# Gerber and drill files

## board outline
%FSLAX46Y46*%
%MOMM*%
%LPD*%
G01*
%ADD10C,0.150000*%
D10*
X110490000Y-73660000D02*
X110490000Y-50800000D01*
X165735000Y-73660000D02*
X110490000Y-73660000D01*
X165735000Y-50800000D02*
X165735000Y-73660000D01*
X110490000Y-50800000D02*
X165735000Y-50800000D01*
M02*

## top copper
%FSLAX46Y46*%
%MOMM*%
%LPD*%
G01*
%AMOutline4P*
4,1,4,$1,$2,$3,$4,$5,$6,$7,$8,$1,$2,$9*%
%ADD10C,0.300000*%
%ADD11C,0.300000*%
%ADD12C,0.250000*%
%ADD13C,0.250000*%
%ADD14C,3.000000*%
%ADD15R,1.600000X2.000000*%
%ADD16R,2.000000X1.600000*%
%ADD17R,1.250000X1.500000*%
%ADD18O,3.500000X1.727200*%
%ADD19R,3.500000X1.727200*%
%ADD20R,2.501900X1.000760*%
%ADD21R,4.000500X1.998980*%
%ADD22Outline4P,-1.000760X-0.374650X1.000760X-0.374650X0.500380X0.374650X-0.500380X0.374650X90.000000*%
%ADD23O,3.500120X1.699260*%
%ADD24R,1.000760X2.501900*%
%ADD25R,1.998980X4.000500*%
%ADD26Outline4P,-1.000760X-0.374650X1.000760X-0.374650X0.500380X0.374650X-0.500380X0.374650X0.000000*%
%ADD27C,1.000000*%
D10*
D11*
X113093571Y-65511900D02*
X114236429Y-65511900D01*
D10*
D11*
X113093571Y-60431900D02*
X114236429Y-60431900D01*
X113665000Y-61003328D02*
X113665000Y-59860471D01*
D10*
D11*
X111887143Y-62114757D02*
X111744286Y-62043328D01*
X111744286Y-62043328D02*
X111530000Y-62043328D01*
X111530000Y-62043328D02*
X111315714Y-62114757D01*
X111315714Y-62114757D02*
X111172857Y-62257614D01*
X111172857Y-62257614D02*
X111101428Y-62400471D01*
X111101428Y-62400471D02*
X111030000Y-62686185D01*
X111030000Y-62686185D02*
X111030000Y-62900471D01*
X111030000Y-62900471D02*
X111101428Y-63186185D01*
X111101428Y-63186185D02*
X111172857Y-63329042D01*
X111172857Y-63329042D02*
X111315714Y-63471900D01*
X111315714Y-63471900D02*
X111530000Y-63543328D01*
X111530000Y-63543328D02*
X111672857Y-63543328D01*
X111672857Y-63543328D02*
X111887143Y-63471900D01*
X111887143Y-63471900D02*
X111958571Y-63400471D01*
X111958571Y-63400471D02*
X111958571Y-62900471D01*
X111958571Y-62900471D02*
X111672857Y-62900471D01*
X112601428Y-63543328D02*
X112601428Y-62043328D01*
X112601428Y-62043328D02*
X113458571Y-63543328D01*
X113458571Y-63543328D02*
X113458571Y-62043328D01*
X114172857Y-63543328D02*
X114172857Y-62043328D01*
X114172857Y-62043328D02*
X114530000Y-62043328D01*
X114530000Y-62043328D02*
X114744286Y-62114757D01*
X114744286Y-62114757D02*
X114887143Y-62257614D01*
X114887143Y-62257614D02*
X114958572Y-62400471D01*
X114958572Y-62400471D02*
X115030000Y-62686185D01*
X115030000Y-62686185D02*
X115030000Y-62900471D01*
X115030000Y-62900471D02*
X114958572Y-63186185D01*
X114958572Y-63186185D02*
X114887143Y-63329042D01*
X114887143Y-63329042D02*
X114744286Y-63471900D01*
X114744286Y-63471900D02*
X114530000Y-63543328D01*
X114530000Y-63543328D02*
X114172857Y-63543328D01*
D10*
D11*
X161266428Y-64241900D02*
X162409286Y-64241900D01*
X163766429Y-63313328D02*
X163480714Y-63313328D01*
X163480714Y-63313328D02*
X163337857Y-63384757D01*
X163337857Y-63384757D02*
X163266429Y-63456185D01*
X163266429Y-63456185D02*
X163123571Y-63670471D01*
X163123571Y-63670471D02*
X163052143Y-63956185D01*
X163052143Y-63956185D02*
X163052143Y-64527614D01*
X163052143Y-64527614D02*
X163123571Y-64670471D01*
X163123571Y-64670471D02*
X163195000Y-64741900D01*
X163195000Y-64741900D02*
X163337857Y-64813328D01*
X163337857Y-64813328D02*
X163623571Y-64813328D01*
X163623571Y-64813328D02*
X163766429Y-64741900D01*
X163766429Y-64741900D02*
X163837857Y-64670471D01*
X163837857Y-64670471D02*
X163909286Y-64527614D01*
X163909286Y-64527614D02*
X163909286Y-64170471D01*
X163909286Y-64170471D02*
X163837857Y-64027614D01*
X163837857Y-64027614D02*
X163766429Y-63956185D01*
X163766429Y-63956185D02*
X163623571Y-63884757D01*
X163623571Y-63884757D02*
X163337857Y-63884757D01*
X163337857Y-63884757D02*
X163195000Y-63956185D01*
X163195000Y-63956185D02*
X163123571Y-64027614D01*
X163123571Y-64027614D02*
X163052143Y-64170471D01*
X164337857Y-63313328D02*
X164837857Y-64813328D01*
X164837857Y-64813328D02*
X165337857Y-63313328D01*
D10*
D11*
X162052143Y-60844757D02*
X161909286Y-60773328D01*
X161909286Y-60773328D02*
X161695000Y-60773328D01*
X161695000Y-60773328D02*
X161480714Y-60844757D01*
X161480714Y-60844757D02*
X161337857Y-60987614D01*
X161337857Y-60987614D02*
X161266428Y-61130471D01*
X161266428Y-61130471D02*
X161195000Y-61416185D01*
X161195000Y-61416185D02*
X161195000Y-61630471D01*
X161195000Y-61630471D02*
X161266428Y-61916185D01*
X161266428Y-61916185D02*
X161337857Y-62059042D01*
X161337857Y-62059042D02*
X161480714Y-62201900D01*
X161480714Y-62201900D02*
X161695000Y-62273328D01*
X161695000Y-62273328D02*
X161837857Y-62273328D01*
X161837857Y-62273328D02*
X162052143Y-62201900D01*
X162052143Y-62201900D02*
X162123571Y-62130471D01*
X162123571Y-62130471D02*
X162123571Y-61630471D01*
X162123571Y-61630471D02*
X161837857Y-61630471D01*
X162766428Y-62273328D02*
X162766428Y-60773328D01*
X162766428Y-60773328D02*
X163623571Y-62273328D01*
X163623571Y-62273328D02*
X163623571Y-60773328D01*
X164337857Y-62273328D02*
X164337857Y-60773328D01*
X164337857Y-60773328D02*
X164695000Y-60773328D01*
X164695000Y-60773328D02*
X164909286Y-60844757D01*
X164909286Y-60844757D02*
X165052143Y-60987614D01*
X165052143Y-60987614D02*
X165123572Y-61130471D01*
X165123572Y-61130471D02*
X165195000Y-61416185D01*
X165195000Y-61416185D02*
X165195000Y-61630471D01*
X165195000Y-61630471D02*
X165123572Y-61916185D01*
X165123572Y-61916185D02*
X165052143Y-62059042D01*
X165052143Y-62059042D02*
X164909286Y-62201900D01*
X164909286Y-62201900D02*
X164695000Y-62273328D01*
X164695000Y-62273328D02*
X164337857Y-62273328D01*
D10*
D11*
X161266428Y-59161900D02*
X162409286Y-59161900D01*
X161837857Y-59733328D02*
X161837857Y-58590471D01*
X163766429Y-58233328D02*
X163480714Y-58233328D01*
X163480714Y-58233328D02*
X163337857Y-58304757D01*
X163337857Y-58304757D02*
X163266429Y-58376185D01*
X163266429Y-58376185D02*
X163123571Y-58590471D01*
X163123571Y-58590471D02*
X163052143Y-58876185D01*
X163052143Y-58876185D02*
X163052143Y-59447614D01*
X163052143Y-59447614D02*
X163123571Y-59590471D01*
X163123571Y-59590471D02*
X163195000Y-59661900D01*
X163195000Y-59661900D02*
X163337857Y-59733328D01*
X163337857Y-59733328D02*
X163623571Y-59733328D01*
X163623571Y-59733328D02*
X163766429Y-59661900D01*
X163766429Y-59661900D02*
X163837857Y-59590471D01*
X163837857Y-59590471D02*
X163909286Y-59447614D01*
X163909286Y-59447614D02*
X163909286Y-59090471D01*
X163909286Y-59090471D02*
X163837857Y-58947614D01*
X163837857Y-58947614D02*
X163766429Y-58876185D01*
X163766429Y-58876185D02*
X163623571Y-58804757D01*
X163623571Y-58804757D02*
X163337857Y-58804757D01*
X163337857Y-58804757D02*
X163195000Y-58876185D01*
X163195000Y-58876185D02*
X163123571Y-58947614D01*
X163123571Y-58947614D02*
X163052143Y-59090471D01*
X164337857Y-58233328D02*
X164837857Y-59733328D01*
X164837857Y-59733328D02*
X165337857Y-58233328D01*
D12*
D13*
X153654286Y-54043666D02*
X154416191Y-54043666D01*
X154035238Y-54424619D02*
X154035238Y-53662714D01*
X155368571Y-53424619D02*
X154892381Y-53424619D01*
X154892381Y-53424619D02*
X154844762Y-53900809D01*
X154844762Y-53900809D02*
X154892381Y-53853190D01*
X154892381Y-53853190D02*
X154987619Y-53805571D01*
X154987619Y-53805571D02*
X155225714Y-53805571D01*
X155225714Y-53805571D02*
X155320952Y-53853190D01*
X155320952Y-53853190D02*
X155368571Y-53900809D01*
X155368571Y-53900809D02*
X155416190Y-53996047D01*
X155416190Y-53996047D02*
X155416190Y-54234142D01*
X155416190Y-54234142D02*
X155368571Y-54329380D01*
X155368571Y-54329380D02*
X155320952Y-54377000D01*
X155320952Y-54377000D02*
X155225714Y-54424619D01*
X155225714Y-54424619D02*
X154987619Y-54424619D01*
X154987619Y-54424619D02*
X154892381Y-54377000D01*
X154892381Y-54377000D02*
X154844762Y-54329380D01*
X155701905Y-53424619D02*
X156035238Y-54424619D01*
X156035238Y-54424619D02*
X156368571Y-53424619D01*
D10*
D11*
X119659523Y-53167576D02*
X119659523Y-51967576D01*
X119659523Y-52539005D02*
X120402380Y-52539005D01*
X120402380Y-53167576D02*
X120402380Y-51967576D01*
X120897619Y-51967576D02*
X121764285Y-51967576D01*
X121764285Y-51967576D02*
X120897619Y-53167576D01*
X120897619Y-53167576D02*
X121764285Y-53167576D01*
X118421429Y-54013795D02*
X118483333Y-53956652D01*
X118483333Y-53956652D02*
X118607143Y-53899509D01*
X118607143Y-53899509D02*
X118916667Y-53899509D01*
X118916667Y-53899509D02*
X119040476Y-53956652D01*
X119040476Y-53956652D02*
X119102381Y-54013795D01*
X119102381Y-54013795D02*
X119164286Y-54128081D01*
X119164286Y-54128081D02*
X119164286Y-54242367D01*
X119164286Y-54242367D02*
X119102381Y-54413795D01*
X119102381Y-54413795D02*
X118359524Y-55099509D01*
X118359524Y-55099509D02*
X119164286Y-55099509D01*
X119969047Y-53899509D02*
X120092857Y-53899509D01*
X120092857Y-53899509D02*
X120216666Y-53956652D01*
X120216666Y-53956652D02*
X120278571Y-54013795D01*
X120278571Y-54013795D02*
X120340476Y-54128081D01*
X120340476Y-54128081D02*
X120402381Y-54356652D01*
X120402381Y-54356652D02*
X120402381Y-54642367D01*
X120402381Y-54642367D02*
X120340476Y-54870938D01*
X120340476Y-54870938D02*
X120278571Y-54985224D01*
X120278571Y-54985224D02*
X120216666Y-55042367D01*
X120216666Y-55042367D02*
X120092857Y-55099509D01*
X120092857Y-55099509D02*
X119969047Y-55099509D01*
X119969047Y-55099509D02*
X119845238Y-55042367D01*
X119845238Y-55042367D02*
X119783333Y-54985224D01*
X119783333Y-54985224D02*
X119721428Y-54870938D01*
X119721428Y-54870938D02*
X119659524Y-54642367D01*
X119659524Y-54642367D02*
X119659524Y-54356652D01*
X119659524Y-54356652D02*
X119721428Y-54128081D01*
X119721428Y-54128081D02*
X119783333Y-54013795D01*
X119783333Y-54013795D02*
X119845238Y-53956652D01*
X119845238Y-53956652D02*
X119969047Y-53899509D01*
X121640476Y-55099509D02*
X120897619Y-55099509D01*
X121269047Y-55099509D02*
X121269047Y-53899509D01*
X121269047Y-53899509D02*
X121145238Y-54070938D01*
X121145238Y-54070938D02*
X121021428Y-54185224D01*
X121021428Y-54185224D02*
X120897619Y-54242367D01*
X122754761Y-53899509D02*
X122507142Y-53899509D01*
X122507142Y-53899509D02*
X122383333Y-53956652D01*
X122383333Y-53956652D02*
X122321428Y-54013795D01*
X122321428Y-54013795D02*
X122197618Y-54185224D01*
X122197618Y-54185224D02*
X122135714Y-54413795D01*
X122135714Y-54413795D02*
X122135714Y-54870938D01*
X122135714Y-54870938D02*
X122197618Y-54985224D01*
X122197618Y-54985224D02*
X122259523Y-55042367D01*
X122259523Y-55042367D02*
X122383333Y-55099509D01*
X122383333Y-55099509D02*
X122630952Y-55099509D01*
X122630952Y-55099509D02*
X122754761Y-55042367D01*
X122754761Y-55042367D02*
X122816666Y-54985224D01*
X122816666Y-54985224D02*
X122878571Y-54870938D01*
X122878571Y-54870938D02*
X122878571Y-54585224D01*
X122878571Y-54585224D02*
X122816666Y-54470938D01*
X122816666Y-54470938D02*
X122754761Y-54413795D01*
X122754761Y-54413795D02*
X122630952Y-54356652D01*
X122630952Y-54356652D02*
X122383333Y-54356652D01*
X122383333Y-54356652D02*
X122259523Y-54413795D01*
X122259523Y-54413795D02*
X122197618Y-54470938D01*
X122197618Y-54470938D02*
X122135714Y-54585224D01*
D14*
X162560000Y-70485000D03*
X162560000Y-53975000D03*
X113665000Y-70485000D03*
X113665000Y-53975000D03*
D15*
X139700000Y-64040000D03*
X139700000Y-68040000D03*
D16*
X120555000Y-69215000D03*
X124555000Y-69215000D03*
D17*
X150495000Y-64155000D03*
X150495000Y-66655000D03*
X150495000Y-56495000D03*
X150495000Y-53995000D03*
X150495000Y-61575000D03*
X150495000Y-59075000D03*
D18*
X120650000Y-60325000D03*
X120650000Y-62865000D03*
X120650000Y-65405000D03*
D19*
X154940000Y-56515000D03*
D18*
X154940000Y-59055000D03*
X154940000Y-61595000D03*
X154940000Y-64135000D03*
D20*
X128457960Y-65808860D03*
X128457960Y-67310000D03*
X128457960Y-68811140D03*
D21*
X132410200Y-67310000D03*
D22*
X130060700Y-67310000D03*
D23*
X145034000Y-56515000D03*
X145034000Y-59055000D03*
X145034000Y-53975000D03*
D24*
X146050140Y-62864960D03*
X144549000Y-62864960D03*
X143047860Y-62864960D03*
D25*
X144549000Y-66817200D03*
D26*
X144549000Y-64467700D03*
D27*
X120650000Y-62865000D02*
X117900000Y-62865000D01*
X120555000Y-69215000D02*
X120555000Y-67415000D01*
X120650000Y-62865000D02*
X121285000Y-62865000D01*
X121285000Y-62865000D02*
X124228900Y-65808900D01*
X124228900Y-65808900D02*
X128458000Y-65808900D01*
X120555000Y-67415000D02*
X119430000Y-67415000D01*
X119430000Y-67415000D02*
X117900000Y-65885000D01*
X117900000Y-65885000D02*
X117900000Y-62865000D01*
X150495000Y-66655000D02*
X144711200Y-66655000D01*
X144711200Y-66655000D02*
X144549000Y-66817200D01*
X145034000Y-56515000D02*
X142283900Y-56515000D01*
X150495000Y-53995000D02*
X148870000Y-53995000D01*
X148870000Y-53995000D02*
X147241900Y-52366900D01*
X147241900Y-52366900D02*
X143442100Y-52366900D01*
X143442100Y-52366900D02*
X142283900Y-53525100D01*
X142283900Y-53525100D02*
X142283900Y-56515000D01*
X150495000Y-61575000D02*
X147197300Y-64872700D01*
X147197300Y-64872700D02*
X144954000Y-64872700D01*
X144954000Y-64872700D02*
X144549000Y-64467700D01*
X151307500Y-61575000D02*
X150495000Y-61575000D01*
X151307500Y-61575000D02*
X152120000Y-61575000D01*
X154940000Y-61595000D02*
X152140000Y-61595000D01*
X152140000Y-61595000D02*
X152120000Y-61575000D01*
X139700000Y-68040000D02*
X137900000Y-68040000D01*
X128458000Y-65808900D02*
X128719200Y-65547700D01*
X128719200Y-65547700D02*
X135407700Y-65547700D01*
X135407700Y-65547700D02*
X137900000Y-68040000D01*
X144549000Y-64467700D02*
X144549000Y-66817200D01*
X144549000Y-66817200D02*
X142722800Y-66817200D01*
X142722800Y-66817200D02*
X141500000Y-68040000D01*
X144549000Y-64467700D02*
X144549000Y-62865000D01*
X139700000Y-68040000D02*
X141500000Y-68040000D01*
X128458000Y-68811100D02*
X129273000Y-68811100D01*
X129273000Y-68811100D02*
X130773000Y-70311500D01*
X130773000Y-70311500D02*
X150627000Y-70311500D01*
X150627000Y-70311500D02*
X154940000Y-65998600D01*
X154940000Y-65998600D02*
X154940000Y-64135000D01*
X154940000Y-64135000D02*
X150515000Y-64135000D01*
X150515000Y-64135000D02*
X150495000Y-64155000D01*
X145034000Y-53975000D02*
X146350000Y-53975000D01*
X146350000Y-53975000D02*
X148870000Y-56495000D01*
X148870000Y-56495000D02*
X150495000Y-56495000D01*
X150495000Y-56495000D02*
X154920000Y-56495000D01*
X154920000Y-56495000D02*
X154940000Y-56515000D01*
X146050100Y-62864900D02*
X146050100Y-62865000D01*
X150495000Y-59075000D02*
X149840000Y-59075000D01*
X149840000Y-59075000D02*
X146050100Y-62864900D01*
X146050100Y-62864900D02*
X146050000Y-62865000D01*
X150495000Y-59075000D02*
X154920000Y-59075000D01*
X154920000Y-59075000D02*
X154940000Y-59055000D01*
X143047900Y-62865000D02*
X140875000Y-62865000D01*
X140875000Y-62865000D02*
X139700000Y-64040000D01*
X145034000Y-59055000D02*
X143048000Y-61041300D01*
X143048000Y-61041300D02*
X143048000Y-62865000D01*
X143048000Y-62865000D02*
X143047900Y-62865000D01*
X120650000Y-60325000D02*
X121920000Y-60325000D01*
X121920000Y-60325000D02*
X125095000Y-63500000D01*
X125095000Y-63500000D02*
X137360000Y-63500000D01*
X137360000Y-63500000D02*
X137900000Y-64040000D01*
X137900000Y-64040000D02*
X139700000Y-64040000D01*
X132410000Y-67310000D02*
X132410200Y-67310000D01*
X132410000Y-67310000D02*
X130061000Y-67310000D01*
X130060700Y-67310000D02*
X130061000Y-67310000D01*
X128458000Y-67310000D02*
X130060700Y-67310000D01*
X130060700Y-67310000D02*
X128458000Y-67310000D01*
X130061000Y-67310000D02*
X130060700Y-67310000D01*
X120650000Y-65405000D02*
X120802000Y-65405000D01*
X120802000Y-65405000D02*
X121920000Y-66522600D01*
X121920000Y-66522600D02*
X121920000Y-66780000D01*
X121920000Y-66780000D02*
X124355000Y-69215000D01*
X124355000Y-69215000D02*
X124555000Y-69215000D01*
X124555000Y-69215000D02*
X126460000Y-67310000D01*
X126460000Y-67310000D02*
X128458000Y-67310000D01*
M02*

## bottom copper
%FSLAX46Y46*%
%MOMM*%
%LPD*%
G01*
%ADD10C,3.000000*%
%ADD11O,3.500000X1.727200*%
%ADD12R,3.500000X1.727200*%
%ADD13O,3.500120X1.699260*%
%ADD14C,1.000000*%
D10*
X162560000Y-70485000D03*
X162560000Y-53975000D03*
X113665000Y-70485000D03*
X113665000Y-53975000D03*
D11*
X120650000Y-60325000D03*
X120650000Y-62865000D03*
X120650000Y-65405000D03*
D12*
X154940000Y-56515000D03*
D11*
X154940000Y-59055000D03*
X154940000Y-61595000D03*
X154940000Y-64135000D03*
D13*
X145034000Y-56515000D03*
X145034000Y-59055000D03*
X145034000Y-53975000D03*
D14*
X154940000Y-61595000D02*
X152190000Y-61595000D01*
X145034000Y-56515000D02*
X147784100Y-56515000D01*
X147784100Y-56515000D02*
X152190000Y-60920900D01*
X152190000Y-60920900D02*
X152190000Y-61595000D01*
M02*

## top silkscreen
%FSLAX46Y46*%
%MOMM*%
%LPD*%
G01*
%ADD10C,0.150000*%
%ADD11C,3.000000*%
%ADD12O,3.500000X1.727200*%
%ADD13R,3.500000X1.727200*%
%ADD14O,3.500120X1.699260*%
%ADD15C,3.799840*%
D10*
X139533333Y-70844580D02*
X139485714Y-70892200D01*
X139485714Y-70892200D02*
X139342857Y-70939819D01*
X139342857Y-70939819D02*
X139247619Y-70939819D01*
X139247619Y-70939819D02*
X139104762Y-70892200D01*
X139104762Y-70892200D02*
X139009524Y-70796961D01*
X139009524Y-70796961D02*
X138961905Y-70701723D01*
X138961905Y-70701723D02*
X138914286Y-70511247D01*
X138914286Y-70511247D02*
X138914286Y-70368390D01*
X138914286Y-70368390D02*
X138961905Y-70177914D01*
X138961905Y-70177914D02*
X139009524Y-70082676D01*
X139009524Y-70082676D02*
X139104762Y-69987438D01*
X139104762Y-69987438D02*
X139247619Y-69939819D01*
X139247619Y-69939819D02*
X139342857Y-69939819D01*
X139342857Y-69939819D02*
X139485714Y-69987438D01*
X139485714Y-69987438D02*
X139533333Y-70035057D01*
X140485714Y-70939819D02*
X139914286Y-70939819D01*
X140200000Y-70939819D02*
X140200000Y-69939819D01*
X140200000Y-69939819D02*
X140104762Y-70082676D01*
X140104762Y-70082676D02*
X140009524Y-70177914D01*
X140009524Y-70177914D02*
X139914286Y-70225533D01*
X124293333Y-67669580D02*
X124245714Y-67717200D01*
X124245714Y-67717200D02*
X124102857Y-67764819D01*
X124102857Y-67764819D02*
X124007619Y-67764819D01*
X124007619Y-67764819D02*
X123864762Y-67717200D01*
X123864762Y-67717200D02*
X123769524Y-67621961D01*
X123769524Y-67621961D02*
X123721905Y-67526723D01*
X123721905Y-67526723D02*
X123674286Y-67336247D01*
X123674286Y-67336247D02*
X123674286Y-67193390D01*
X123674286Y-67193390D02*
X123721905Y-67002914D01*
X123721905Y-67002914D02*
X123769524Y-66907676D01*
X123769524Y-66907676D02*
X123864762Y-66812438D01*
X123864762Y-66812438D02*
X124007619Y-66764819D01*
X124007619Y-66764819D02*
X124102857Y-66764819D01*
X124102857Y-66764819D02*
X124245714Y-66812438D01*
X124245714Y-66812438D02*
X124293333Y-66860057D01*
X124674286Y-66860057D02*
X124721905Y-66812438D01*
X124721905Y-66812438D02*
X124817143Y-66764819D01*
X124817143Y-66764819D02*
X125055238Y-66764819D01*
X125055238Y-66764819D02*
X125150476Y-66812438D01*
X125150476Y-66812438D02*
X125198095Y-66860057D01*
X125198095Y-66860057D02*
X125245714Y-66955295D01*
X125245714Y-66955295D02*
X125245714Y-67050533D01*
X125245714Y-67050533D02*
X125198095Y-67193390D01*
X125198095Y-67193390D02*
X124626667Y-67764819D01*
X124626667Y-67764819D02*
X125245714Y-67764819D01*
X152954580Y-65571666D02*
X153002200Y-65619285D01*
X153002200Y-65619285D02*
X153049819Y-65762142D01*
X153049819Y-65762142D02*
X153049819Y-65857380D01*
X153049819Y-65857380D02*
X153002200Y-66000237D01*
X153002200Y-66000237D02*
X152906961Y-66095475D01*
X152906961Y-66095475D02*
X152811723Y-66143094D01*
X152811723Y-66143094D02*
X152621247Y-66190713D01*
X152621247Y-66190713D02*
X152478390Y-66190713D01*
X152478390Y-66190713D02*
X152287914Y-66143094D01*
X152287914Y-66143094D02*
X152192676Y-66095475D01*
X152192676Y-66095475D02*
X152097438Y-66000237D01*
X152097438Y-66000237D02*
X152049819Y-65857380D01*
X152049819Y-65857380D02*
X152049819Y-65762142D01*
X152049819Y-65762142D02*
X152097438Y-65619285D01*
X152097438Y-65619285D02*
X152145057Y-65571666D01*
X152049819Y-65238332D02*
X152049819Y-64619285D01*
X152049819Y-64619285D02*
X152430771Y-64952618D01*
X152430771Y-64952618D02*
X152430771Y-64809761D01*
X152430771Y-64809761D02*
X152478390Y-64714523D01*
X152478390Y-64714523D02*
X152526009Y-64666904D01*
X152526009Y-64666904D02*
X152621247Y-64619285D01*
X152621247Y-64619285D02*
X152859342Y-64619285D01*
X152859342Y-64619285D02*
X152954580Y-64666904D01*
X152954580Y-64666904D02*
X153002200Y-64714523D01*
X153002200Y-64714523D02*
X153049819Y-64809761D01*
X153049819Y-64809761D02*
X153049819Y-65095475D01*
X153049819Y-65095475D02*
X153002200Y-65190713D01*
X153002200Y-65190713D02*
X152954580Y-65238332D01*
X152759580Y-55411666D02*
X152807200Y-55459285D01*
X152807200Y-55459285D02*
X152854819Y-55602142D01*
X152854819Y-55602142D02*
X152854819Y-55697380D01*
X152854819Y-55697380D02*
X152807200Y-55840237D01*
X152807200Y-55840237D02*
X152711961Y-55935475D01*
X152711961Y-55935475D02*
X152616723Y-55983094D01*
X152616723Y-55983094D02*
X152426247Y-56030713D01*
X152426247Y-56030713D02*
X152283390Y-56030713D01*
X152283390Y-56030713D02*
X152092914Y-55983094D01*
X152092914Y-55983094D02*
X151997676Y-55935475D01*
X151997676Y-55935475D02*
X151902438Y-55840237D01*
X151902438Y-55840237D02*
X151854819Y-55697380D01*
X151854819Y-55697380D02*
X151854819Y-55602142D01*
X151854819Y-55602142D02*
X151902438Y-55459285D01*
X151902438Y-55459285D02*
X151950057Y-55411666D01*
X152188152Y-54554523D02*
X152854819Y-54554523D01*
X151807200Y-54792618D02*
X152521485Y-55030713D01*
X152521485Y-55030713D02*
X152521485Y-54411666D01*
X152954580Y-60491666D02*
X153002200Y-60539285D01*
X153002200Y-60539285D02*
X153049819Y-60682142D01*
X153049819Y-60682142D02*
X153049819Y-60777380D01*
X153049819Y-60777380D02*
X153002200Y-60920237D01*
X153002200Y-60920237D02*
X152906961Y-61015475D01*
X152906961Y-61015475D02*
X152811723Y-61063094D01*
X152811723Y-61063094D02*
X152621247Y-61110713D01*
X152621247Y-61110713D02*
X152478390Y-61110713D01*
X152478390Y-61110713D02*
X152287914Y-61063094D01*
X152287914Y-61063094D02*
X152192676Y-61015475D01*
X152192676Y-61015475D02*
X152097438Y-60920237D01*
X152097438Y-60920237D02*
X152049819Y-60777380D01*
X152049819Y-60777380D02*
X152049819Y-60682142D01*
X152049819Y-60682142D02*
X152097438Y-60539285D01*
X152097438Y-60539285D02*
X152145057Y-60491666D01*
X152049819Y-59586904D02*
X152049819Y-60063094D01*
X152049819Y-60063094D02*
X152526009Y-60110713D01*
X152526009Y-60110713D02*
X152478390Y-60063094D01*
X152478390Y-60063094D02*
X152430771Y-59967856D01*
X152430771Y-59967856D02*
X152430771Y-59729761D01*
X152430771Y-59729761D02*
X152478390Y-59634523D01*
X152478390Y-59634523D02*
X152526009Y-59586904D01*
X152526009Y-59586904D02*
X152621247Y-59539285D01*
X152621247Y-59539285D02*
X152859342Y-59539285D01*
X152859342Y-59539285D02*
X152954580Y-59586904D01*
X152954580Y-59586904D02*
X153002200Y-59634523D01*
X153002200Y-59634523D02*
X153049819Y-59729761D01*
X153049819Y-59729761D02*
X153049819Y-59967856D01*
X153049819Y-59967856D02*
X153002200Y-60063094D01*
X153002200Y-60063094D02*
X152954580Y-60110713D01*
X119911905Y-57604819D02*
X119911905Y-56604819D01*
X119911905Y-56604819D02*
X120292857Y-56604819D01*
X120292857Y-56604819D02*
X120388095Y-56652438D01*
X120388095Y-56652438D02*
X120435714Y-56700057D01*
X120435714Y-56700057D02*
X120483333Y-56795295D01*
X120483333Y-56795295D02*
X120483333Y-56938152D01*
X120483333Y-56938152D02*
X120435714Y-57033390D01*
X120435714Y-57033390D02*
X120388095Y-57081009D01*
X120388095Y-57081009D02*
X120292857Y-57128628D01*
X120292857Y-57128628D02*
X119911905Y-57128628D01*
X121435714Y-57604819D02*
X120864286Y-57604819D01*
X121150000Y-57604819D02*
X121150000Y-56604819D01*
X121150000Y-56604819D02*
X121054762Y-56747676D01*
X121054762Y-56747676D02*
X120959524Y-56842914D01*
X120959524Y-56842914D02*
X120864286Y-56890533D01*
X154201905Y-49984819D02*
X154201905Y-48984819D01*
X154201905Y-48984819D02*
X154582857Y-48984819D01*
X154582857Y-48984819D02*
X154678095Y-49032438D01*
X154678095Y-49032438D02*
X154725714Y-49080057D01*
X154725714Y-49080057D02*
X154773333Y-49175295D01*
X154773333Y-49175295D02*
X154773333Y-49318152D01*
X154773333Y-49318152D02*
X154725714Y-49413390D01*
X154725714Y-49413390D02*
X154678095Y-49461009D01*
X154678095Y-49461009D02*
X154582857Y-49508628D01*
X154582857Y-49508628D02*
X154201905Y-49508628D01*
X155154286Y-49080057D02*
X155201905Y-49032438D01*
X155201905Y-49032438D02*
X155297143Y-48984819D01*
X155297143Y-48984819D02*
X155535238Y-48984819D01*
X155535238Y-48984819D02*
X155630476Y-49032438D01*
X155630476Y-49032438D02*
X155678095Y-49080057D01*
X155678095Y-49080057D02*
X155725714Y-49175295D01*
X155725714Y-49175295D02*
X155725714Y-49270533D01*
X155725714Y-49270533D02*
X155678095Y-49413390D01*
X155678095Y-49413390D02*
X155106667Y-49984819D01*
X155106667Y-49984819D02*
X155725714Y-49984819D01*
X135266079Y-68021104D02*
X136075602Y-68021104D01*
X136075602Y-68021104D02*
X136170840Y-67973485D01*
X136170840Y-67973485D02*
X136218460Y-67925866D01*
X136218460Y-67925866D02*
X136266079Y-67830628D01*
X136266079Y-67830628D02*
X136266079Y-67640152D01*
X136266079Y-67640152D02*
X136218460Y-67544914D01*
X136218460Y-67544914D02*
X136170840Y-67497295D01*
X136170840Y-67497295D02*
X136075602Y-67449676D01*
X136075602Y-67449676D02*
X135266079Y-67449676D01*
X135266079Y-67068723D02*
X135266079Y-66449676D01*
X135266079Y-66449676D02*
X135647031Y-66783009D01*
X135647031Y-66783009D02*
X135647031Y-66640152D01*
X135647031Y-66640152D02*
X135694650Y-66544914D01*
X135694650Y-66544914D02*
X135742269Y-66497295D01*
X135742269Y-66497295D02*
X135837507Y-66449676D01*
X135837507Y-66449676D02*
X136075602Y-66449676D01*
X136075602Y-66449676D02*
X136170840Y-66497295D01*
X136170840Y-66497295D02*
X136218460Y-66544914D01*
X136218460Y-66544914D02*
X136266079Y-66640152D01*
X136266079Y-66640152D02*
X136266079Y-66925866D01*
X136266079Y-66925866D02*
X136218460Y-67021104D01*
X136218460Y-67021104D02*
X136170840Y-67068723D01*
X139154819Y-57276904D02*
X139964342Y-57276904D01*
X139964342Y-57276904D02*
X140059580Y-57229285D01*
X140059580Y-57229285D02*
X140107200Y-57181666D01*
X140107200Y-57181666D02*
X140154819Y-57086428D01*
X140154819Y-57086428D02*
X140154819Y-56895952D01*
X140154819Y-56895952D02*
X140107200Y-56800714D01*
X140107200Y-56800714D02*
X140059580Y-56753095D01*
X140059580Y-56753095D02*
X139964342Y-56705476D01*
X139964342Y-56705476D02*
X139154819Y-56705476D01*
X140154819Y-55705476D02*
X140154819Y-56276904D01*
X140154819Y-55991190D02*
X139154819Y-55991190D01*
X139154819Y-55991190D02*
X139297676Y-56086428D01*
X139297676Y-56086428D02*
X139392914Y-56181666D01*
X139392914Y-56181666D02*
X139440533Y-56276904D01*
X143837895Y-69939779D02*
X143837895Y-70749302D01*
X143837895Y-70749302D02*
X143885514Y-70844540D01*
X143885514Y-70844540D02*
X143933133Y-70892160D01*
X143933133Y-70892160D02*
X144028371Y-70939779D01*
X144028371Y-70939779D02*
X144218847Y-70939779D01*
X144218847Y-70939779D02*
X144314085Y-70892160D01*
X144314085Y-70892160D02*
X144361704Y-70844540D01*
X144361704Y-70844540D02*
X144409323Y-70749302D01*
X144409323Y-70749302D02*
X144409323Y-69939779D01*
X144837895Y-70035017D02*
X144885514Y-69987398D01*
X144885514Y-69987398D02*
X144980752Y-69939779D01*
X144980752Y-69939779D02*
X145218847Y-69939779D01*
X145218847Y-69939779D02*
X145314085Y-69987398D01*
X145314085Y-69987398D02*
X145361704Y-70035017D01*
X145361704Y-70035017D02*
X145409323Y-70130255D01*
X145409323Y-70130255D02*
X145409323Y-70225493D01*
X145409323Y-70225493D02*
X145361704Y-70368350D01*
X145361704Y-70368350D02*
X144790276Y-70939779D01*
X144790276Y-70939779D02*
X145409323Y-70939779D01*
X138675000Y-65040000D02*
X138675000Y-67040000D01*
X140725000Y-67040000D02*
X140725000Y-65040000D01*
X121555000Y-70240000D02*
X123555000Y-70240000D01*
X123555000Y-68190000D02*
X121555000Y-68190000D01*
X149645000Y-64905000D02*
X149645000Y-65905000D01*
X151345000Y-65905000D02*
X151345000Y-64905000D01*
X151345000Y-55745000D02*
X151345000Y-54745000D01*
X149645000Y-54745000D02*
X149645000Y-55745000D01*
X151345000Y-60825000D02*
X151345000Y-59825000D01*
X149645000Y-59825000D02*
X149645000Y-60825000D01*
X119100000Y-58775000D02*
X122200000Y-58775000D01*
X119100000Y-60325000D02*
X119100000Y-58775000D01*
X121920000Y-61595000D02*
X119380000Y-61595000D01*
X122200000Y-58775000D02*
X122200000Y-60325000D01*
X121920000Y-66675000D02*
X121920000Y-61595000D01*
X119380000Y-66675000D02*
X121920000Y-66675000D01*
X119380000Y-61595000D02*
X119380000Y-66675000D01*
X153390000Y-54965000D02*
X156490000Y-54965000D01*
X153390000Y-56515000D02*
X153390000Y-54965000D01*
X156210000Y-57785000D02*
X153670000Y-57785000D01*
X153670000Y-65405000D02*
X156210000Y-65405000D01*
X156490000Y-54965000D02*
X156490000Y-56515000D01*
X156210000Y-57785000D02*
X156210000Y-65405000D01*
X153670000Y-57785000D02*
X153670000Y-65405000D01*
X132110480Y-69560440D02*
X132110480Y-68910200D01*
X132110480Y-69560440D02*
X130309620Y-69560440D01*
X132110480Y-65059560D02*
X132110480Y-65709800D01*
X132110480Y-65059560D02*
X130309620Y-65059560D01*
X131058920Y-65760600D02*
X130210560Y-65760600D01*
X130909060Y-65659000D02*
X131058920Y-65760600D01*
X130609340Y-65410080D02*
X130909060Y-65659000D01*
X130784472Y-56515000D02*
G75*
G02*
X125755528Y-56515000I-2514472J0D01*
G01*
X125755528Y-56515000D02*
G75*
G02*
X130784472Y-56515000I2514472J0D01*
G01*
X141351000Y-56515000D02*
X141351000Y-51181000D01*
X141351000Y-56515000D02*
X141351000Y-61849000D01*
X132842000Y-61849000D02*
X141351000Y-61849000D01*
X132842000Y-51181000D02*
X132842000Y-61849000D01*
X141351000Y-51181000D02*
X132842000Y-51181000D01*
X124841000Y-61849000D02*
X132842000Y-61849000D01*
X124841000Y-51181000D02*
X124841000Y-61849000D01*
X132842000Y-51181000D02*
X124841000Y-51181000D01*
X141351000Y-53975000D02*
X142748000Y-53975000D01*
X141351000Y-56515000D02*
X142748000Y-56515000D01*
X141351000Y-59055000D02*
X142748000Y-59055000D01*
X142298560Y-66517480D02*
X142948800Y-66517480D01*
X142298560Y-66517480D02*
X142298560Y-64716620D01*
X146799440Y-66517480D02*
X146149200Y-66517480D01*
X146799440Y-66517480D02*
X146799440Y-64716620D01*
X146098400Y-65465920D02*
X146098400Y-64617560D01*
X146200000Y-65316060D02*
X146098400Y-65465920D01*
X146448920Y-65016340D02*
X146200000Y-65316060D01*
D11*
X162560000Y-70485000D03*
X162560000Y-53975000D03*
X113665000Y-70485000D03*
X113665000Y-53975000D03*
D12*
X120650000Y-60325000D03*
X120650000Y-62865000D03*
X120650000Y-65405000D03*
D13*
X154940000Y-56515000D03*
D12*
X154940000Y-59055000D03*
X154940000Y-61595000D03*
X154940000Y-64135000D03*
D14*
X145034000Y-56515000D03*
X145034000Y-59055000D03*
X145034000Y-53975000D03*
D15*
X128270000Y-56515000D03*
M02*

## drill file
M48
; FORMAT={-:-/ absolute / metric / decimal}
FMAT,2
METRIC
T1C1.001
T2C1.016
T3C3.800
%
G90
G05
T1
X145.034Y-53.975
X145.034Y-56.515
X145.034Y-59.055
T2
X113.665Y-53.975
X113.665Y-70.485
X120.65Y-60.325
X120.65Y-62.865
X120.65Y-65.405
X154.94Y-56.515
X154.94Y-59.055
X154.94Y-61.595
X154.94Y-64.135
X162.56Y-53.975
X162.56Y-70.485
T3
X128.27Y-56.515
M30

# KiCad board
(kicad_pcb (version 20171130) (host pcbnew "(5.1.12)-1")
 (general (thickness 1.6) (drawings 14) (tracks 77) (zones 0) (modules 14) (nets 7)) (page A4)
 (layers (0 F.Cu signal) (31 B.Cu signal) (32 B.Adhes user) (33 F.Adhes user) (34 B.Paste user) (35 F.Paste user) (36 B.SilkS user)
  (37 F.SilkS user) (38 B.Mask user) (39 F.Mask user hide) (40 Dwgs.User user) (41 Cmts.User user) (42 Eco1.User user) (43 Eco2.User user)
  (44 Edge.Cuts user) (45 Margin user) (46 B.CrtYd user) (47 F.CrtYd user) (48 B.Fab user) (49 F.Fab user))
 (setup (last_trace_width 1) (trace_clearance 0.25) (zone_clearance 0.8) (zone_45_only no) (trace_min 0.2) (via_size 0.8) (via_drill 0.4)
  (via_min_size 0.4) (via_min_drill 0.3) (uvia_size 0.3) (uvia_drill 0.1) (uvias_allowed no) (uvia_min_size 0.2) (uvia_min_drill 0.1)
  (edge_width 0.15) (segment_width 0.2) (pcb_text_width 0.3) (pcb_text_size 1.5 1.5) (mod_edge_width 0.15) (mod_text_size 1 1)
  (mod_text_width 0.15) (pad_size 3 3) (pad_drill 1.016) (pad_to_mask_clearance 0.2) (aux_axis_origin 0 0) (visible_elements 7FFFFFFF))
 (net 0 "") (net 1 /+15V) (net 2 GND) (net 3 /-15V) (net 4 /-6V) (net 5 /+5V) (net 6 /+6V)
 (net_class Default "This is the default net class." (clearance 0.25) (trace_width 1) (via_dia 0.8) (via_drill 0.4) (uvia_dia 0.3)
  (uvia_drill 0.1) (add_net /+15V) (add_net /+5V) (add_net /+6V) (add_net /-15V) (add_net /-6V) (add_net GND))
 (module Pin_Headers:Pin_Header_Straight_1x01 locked (layer F.Cu) (at 162.56 70.485)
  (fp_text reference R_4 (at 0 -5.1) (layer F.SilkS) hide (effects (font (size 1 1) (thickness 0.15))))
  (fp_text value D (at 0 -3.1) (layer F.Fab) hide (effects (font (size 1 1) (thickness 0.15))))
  (pad 1 thru_hole circle (at 0 0) (size 3 3) (drill 1.016) (layers *.Cu *.Mask F.SilkS)))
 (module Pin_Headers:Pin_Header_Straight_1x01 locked (layer F.Cu) (at 162.56 53.975)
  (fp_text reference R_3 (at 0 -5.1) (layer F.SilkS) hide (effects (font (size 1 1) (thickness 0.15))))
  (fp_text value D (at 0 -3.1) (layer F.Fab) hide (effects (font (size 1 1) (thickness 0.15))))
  (pad 1 thru_hole circle (at 0 0) (size 3 3) (drill 1.016) (layers *.Cu *.Mask F.SilkS)))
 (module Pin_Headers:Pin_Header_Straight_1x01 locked (layer F.Cu) (at 113.665 70.485)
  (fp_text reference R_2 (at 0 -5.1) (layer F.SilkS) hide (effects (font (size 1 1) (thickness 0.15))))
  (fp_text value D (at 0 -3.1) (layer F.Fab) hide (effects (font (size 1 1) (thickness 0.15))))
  (pad 1 thru_hole circle (at 0 0) (size 3 3) (drill 1.016) (layers *.Cu *.Mask F.SilkS)))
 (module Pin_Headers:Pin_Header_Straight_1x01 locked (layer F.Cu) (at 113.665 53.975)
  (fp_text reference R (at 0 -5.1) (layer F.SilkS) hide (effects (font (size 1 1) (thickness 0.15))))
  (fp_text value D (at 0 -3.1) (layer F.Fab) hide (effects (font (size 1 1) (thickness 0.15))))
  (pad 1 thru_hole circle (at 0 0) (size 3 3) (drill 1.016) (layers *.Cu *.Mask F.SilkS)))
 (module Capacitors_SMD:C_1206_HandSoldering (layer F.Cu) (at 139.7 66.04 270)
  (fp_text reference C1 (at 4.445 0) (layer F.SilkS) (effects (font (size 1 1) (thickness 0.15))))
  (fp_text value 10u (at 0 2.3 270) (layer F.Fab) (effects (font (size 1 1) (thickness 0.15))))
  (fp_line (start -1 1.025) (end 1 1.025) (layer F.SilkS) (width 0.15))
  (fp_line (start 1 -1.025) (end -1 -1.025) (layer F.SilkS) (width 0.15))
  (pad 1 smd rect (at -2 0 270) (size 2 1.6) (layers F.Cu F.Paste F.Mask) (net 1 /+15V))
  (pad 2 smd rect (at 2 0 270) (size 2 1.6) (layers F.Cu F.Paste F.Mask) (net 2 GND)))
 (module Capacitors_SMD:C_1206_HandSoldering (layer F.Cu) (at 122.555 69.215 180)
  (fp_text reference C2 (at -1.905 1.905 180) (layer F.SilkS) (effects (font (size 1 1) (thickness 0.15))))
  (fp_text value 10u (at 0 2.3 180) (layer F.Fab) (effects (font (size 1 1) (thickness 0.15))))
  (fp_line (start 1 -1.025) (end -1 -1.025) (layer F.SilkS) (width 0.15))
  (fp_line (start -1 1.025) (end 1 1.025) (layer F.SilkS) (width 0.15))
  (pad 2 smd rect (at 2 0 180) (size 2 1.6) (layers F.Cu F.Paste F.Mask) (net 2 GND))
  (pad 1 smd rect (at -2 0 180) (size 2 1.6) (layers F.Cu F.Paste F.Mask) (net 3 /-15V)))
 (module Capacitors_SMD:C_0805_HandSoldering (layer F.Cu) (at 150.495 65.405 270)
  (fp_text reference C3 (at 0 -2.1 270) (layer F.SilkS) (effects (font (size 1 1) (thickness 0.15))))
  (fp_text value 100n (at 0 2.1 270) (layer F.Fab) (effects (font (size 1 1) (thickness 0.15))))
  (fp_line (start -0.5 0.85) (end 0.5 0.85) (layer F.SilkS) (width 0.15))
  (fp_line (start 0.5 -0.85) (end -0.5 -0.85) (layer F.SilkS) (width 0.15))
  (pad 1 smd rect (at -1.25 0 270) (size 1.5 1.25) (layers F.Cu F.Paste F.Mask) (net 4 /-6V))
  (pad 2 smd rect (at 1.25 0 270) (size 1.5 1.25) (layers F.Cu F.Paste F.Mask) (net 2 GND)))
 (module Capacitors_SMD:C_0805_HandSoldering (layer F.Cu) (at 150.495 55.245 90)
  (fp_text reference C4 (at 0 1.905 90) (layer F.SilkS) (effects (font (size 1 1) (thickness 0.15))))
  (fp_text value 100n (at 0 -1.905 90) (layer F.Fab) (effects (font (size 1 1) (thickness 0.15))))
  (fp_line (start -0.5 0.85) (end 0.5 0.85) (layer F.SilkS) (width 0.15))
  (fp_line (start 0.5 -0.85) (end -0.5 -0.85) (layer F.SilkS) (width 0.15))
  (pad 1 smd rect (at -1.25 0 90) (size 1.5 1.25) (layers F.Cu F.Paste F.Mask) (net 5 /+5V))
  (pad 2 smd rect (at 1.25 0 90) (size 1.5 1.25) (layers F.Cu F.Paste F.Mask) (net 2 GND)))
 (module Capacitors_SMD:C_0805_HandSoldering (layer F.Cu) (at 150.495 60.325 270)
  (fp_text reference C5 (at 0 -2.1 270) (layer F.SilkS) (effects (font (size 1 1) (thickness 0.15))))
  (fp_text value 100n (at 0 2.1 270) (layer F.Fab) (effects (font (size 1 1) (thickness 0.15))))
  (fp_line (start 0.5 -0.85) (end -0.5 -0.85) (layer F.SilkS) (width 0.15))
  (fp_line (start -0.5 0.85) (end 0.5 0.85) (layer F.SilkS) (width 0.15))
  (pad 2 smd rect (at 1.25 0 270) (size 1.5 1.25) (layers F.Cu F.Paste F.Mask) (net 2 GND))
  (pad 1 smd rect (at -1.25 0 270) (size 1.5 1.25) (layers F.Cu F.Paste F.Mask) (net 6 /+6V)))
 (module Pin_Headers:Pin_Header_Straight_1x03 (layer F.Cu) (at 120.65 60.325)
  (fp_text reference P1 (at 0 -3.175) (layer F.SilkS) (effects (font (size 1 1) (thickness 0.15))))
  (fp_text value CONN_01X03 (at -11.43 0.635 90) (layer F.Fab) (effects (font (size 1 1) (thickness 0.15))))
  (fp_line (start -1.55 -1.55) (end 1.55 -1.55) (layer F.SilkS) (width 0.15))
  (fp_line (start -1.55 0) (end -1.55 -1.55) (layer F.SilkS) (width 0.15))
  (fp_line (start 1.27 1.27) (end -1.27 1.27) (layer F.SilkS) (width 0.15))
  (fp_line (start 1.55 -1.55) (end 1.55 0) (layer F.SilkS) (width 0.15))
  (fp_line (start 1.27 6.35) (end 1.27 1.27) (layer F.SilkS) (width 0.15))
  (fp_line (start -1.27 6.35) (end 1.27 6.35) (layer F.SilkS) (width 0.15))
  (fp_line (start -1.27 1.27) (end -1.27 6.35) (layer F.SilkS) (width 0.15))
  (pad 1 thru_hole oval (at 0 0) (size 3.5 1.7272) (drill 1.016) (layers *.Cu *.Mask F.SilkS) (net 1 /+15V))
  (pad 2 thru_hole oval (at 0 2.54) (size 3.5 1.7272) (drill 1.016) (layers *.Cu *.Mask F.SilkS) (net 2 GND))
  (pad 3 thru_hole oval (at 0 5.08) (size 3.5 1.7272) (drill 1.016) (layers *.Cu *.Mask F.SilkS) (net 3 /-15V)))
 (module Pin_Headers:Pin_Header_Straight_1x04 (layer F.Cu) (at 154.94 56.515)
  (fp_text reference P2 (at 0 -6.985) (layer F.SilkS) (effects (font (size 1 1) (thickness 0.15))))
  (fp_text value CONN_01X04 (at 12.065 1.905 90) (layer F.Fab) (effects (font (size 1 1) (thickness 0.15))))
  (fp_line (start -1.55 -1.55) (end 1.55 -1.55) (layer F.SilkS) (width 0.15))
  (fp_line (start -1.55 0) (end -1.55 -1.55) (layer F.SilkS) (width 0.15))
  (fp_line (start 1.27 1.27) (end -1.27 1.27) (layer F.SilkS) (width 0.15))
  (fp_line (start -1.27 8.89) (end 1.27 8.89) (layer F.SilkS) (width 0.15))
  (fp_line (start 1.55 -1.55) (end 1.55 0) (layer F.SilkS) (width 0.15))
  (fp_line (start 1.27 1.27) (end 1.27 8.89) (layer F.SilkS) (width 0.15))
  (fp_line (start -1.27 1.27) (end -1.27 8.89) (layer F.SilkS) (width 0.15))
  (pad 1 thru_hole rect (at 0 0) (size 3.5 1.7272) (drill 1.016) (layers *.Cu *.Mask F.SilkS) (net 5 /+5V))
  (pad 2 thru_hole oval (at 0 2.54) (size 3.5 1.7272) (drill 1.016) (layers *.Cu *.Mask F.SilkS) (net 6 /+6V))
  (pad 3 thru_hole oval (at 0 5.08) (size 3.5 1.7272) (drill 1.016) (layers *.Cu *.Mask F.SilkS) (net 2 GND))
  (pad 4 thru_hole oval (at 0 7.62) (size 3.5 1.7272) (drill 1.016) (layers *.Cu *.Mask F.SilkS) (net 4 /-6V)))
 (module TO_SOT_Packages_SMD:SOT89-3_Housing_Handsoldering (layer F.Cu) (at 130.81 67.31 270)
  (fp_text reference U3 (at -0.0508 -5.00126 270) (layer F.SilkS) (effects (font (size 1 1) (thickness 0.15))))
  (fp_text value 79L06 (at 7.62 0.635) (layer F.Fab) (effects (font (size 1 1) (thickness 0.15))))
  (fp_line (start 2.25044 -1.30048) (end 1.6002 -1.30048) (layer F.SilkS) (width 0.15))
  (fp_line (start 2.25044 -1.30048) (end 2.25044 0.50038) (layer F.SilkS) (width 0.15))
  (fp_line (start -2.25044 -1.30048) (end -1.6002 -1.30048) (layer F.SilkS) (width 0.15))
  (fp_line (start -2.25044 -1.30048) (end -2.25044 0.50038) (layer F.SilkS) (width 0.15))
  (fp_line (start -1.5494 -0.24892) (end -1.5494 0.59944) (layer F.SilkS) (width 0.15))
  (fp_line (start -1.651 -0.09906) (end -1.5494 -0.24892) (layer F.SilkS) (width 0.15))
  (fp_line (start -1.89992 0.20066) (end -1.651 -0.09906) (layer F.SilkS) (width 0.15))
  (pad 1 smd rect (at -1.50114 2.35204 270) (size 1.00076 2.5019) (layers F.Cu F.Paste F.Mask) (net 2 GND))
  (pad 2 smd rect (at 0 2.35204 270) (size 1.00076 2.5019) (layers F.Cu F.Paste F.Mask) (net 3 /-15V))
  (pad 3 smd rect (at 1.50114 2.35204 270) (size 1.00076 2.5019) (layers F.Cu F.Paste F.Mask) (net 4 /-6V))
  (pad 2 smd rect (at 0 -1.6002 270) (size 1.99898 4.0005) (layers F.Cu F.Paste F.Mask) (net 3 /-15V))
  (pad 2 smd trapezoid (at 0 0.7493 90) (size 1.50114 0.7493) (rect_delta 0 0.50038) (layers F.Cu F.Paste F.Mask) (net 3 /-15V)))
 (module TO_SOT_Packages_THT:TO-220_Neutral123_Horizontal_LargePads (layer F.Cu) (at 145.034 56.515 90)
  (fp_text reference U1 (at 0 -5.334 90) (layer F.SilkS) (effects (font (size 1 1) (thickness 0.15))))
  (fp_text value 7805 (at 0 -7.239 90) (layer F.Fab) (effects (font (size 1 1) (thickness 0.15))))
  (fp_circle (center 0 -16.764) (end 1.778 -14.986) (layer F.SilkS) (width 0.15))
  (fp_line (start 0 -3.683) (end 5.334 -3.683) (layer F.SilkS) (width 0.15))
  (fp_line (start 0 -3.683) (end -5.334 -3.683) (layer F.SilkS) (width 0.15))
  (fp_line (start -5.334 -12.192) (end -5.334 -3.683) (layer F.SilkS) (width 0.15))
  (fp_line (start 5.334 -12.192) (end -5.334 -12.192) (layer F.SilkS) (width 0.15))
  (fp_line (start 5.334 -3.683) (end 5.334 -12.192) (layer F.SilkS) (width 0.15))
  (fp_line (start -5.334 -20.193) (end -5.334 -12.192) (layer F.SilkS) (width 0.15))
  (fp_line (start 5.334 -20.193) (end -5.334 -20.193) (layer F.SilkS) (width 0.15))
  (fp_line (start 5.334 -12.192) (end 5.334 -20.193) (layer F.SilkS) (width 0.15))
  (fp_line (start 2.54 -3.683) (end 2.54 -2.286) (layer F.SilkS) (width 0.15))
  (fp_line (start 0 -3.683) (end 0 -2.286) (layer F.SilkS) (width 0.15))
  (fp_line (start -2.54 -3.683) (end -2.54 -2.286) (layer F.SilkS) (width 0.15))
  (pad 2 thru_hole oval (at 0 0 180) (size 3.50012 1.69926) (drill 1.00076) (layers *.Cu *.Mask F.SilkS) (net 2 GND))
  (pad 1 thru_hole oval (at -2.54 0 180) (size 3.50012 1.69926) (drill 1.00076) (layers *.Cu *.Mask F.SilkS) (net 1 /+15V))
  (pad 3 thru_hole oval (at 2.54 0 180) (size 3.50012 1.69926) (drill 1.00076) (layers *.Cu *.Mask F.SilkS) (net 5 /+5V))
  (pad "" np_thru_hole circle (at 0 -16.764 180) (size 3.79984 3.79984) (drill 3.79984) (layers *.Cu *.Mask F.SilkS)))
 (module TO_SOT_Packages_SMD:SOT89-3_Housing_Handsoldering (layer F.Cu) (at 144.549 65.217 180)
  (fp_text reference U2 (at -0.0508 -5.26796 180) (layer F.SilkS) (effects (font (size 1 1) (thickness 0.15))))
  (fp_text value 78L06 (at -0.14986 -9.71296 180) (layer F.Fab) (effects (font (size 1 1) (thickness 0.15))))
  (fp_line (start 2.25044 -1.30048) (end 1.6002 -1.30048) (layer F.SilkS) (width 0.15))
  (fp_line (start 2.25044 -1.30048) (end 2.25044 0.50038) (layer F.SilkS) (width 0.15))
  (fp_line (start -2.25044 -1.30048) (end -1.6002 -1.30048) (layer F.SilkS) (width 0.15))
  (fp_line (start -2.25044 -1.30048) (end -2.25044 0.50038) (layer F.SilkS) (width 0.15))
  (fp_line (start -1.5494 -0.24892) (end -1.5494 0.59944) (layer F.SilkS) (width 0.15))
  (fp_line (start -1.651 -0.09906) (end -1.5494 -0.24892) (layer F.SilkS) (width 0.15))
  (fp_line (start -1.89992 0.20066) (end -1.651 -0.09906) (layer F.SilkS) (width 0.15))
  (pad 1 smd rect (at -1.50114 2.35204 180) (size 1.00076 2.5019) (layers F.Cu F.Paste F.Mask) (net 6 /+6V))
  (pad 2 smd rect (at 0 2.35204 180) (size 1.00076 2.5019) (layers F.Cu F.Paste F.Mask) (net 2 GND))
  (pad 3 smd rect (at 1.50114 2.35204 180) (size 1.00076 2.5019) (layers F.Cu F.Paste F.Mask) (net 1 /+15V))
  (pad 2 smd rect (at 0 -1.6002 180) (size 1.99898 4.0005) (layers F.Cu F.Paste F.Mask) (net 2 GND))
  (pad 2 smd trapezoid (at 0 0.7493) (size 1.50114 0.7493) (rect_delta 0 0.50038) (layers F.Cu F.Paste F.Mask) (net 2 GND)))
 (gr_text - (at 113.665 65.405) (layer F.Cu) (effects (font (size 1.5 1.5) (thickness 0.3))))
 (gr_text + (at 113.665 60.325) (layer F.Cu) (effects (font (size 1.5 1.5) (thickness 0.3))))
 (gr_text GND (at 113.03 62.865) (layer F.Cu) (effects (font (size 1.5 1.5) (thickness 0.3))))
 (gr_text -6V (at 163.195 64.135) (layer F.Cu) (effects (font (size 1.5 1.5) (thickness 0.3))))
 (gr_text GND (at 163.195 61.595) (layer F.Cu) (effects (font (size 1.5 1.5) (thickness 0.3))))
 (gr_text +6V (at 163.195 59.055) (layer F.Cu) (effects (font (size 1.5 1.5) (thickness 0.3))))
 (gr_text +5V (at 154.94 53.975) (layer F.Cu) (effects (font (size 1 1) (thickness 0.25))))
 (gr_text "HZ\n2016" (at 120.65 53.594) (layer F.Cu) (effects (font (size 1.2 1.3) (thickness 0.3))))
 (gr_line (start 110.49 73.66) (end 110.49 50.8) (layer Edge.Cuts) (width 0.15))
 (gr_line (start 165.735 73.66) (end 110.49 73.66) (layer Edge.Cuts) (width 0.15))
 (gr_line (start 165.735 50.8) (end 165.735 73.66) (layer Edge.Cuts) (width 0.15))
 (gr_line (start 110.49 50.8) (end 165.735 50.8) (layer Edge.Cuts) (width 0.15))
 (segment (start 120.65 62.865) (end 117.9 62.865) (width 1) (layer F.Cu) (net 2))
 (segment (start 120.555 69.215) (end 120.555 67.415) (width 1) (layer F.Cu) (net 2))
 (segment (start 120.65 62.865) (end 121.285 62.865) (width 1) (layer F.Cu) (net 2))
 (segment (start 121.285 62.865) (end 124.2289 65.8089) (width 1) (layer F.Cu) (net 2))
 (segment (start 124.2289 65.8089) (end 128.458 65.8089) (width 1) (layer F.Cu) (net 2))
 (segment (start 120.555 67.415) (end 119.43 67.415) (width 1) (layer F.Cu) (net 2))
 (segment (start 119.43 67.415) (end 117.9 65.885) (width 1) (layer F.Cu) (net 2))
 (segment (start 117.9 65.885) (end 117.9 62.865) (width 1) (layer F.Cu) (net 2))
 (segment (start 150.495 66.655) (end 144.7112 66.655) (width 1) (layer F.Cu) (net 2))
 (segment (start 144.7112 66.655) (end 144.549 66.8172) (width 1) (layer F.Cu) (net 2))
 (segment (start 145.034 56.515) (end 142.2839 56.515) (width 1) (layer F.Cu) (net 2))
 (segment (start 150.495 53.995) (end 148.87 53.995) (width 1) (layer F.Cu) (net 2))
 (segment (start 148.87 53.995) (end 147.2419 52.3669) (width 1) (layer F.Cu) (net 2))
 (segment (start 147.2419 52.3669) (end 143.4421 52.3669) (width 1) (layer F.Cu) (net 2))
 (segment (start 143.4421 52.3669) (end 142.2839 53.5251) (width 1) (layer F.Cu) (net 2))
 (segment (start 142.2839 53.5251) (end 142.2839 56.515) (width 1) (layer F.Cu) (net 2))
 (segment (start 150.495 61.575) (end 147.1973 64.8727) (width 1) (layer F.Cu) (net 2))
 (segment (start 147.1973 64.8727) (end 144.954 64.8727) (width 1) (layer F.Cu) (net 2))
 (segment (start 144.954 64.8727) (end 144.549 64.4677) (width 1) (layer F.Cu) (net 2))
 (segment (start 151.3075 61.575) (end 150.495 61.575) (width 1) (layer F.Cu) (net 2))
 (segment (start 151.3075 61.575) (end 152.12 61.575) (width 1) (layer F.Cu) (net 2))
 (segment (start 154.94 61.595) (end 152.14 61.595) (width 1) (layer F.Cu) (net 2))
 (segment (start 152.14 61.595) (end 152.12 61.575) (width 1) (layer F.Cu) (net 2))
 (segment (start 139.7 68.04) (end 137.9 68.04) (width 1) (layer F.Cu) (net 2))
 (segment (start 128.458 65.8089) (end 128.7192 65.5477) (width 1) (layer F.Cu) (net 2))
 (segment (start 128.7192 65.5477) (end 135.4077 65.5477) (width 1) (layer F.Cu) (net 2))
 (segment (start 135.4077 65.5477) (end 137.9 68.04) (width 1) (layer F.Cu) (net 2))
 (segment (start 144.549 64.4677) (end 144.549 66.8172) (width 1) (layer F.Cu) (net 2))
 (segment (start 144.549 66.8172) (end 142.7228 66.8172) (width 1) (layer F.Cu) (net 2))
 (segment (start 142.7228 66.8172) (end 141.5 68.04) (width 1) (layer F.Cu) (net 2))
 (segment (start 144.549 64.4677) (end 144.549 62.865) (width 1) (layer F.Cu) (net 2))
 (segment (start 139.7 68.04) (end 141.5 68.04) (width 1) (layer F.Cu) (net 2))
 (segment (start 154.94 61.595) (end 152.19 61.595) (width 1) (layer B.Cu) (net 2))
 (segment (start 145.034 56.515) (end 147.7841 56.515) (width 1) (layer B.Cu) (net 2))
 (segment (start 147.7841 56.515) (end 152.19 60.9209) (width 1) (layer B.Cu) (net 2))
 (segment (start 152.19 60.9209) (end 152.19 61.595) (width 1) (layer B.Cu) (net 2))
 (segment (start 128.458 68.8111) (end 129.273 68.8111) (width 1) (layer F.Cu) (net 4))
 (segment (start 129.273 68.8111) (end 130.773 70.3115) (width 1) (layer F.Cu) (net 4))
 (segment (start 130.773 70.3115) (end 150.627 70.3115) (width 1) (layer F.Cu) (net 4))
 (segment (start 150.627 70.3115) (end 154.94 65.9986) (width 1) (layer F.Cu) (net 4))
 (segment (start 154.94 65.9986) (end 154.94 64.135) (width 1) (layer F.Cu) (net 4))
 (segment (start 154.94 64.135) (end 150.515 64.135) (width 1) (layer F.Cu) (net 4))
 (segment (start 150.515 64.135) (end 150.495 64.155) (width 1) (layer F.Cu) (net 4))
 (segment (start 145.034 53.975) (end 146.35 53.975) (width 1) (layer F.Cu) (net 5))
 (segment (start 146.35 53.975) (end 148.87 56.495) (width 1) (layer F.Cu) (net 5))
 (segment (start 148.87 56.495) (end 150.495 56.495) (width 1) (layer F.Cu) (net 5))
 (segment (start 150.495 56.495) (end 154.92 56.495) (width 1) (layer F.Cu) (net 5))
 (segment (start 154.92 56.495) (end 154.94 56.515) (width 1) (layer F.Cu) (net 5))
 (segment (start 146.0501 62.8649) (end 146.0501 62.865) (width 1) (layer F.Cu) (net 6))
 (segment (start 150.495 59.075) (end 149.84 59.075) (width 1) (layer F.Cu) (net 6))
 (segment (start 149.84 59.075) (end 146.0501 62.8649) (width 1) (layer F.Cu) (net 6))
 (segment (start 146.0501 62.8649) (end 146.05 62.865) (width 1) (layer F.Cu) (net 6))
 (segment (start 150.495 59.075) (end 154.92 59.075) (width 1) (layer F.Cu) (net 6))
 (segment (start 154.92 59.075) (end 154.94 59.055) (width 1) (layer F.Cu) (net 6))
 (segment (start 143.0479 62.865) (end 140.875 62.865) (width 1) (layer F.Cu) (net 1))
 (segment (start 140.875 62.865) (end 139.7 64.04) (width 1) (layer F.Cu) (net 1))
 (segment (start 145.034 59.055) (end 143.048 61.0413) (width 1) (layer F.Cu) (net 1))
 (segment (start 143.048 61.0413) (end 143.048 62.865) (width 1) (layer F.Cu) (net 1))
 (segment (start 143.048 62.865) (end 143.0479 62.865) (width 1) (layer F.Cu) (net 1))
 (segment (start 120.65 60.325) (end 121.92 60.325) (width 1) (layer F.Cu) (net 1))
 (segment (start 121.92 60.325) (end 125.095 63.5) (width 1) (layer F.Cu) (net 1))
 (segment (start 125.095 63.5) (end 137.36 63.5) (width 1) (layer F.Cu) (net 1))
 (segment (start 137.36 63.5) (end 137.9 64.04) (width 1) (layer F.Cu) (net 1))
 (segment (start 137.9 64.04) (end 139.7 64.04) (width 1) (layer F.Cu) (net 1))
 (segment (start 132.41 67.31) (end 132.4102 67.31) (width 1) (layer F.Cu) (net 3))
 (segment (start 132.41 67.31) (end 130.061 67.31) (width 1) (layer F.Cu) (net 3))
 (segment (start 130.0607 67.31) (end 130.061 67.31) (width 1) (layer F.Cu) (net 3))
 (segment (start 128.458 67.31) (end 130.0607 67.31) (width 1) (layer F.Cu) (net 3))
 (segment (start 130.0607 67.31) (end 128.458 67.31) (width 1) (layer F.Cu) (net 3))
 (segment (start 130.061 67.31) (end 130.0607 67.31) (width 1) (layer F.Cu) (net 3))
 (segment (start 120.65 65.405) (end 120.802 65.405) (width 1) (layer F.Cu) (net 3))
 (segment (start 120.802 65.405) (end 121.92 66.5226) (width 1) (layer F.Cu) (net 3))
 (segment (start 121.92 66.5226) (end 121.92 66.78) (width 1) (layer F.Cu) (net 3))
 (segment (start 121.92 66.78) (end 124.355 69.215) (width 1) (layer F.Cu) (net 3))
 (segment (start 124.355 69.215) (end 124.555 69.215) (width 1) (layer F.Cu) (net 3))
 (segment (start 124.555 69.215) (end 126.46 67.31) (width 1) (layer F.Cu) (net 3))
 (segment (start 126.46 67.31) (end 128.458 67.31) (width 1) (layer F.Cu) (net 3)))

